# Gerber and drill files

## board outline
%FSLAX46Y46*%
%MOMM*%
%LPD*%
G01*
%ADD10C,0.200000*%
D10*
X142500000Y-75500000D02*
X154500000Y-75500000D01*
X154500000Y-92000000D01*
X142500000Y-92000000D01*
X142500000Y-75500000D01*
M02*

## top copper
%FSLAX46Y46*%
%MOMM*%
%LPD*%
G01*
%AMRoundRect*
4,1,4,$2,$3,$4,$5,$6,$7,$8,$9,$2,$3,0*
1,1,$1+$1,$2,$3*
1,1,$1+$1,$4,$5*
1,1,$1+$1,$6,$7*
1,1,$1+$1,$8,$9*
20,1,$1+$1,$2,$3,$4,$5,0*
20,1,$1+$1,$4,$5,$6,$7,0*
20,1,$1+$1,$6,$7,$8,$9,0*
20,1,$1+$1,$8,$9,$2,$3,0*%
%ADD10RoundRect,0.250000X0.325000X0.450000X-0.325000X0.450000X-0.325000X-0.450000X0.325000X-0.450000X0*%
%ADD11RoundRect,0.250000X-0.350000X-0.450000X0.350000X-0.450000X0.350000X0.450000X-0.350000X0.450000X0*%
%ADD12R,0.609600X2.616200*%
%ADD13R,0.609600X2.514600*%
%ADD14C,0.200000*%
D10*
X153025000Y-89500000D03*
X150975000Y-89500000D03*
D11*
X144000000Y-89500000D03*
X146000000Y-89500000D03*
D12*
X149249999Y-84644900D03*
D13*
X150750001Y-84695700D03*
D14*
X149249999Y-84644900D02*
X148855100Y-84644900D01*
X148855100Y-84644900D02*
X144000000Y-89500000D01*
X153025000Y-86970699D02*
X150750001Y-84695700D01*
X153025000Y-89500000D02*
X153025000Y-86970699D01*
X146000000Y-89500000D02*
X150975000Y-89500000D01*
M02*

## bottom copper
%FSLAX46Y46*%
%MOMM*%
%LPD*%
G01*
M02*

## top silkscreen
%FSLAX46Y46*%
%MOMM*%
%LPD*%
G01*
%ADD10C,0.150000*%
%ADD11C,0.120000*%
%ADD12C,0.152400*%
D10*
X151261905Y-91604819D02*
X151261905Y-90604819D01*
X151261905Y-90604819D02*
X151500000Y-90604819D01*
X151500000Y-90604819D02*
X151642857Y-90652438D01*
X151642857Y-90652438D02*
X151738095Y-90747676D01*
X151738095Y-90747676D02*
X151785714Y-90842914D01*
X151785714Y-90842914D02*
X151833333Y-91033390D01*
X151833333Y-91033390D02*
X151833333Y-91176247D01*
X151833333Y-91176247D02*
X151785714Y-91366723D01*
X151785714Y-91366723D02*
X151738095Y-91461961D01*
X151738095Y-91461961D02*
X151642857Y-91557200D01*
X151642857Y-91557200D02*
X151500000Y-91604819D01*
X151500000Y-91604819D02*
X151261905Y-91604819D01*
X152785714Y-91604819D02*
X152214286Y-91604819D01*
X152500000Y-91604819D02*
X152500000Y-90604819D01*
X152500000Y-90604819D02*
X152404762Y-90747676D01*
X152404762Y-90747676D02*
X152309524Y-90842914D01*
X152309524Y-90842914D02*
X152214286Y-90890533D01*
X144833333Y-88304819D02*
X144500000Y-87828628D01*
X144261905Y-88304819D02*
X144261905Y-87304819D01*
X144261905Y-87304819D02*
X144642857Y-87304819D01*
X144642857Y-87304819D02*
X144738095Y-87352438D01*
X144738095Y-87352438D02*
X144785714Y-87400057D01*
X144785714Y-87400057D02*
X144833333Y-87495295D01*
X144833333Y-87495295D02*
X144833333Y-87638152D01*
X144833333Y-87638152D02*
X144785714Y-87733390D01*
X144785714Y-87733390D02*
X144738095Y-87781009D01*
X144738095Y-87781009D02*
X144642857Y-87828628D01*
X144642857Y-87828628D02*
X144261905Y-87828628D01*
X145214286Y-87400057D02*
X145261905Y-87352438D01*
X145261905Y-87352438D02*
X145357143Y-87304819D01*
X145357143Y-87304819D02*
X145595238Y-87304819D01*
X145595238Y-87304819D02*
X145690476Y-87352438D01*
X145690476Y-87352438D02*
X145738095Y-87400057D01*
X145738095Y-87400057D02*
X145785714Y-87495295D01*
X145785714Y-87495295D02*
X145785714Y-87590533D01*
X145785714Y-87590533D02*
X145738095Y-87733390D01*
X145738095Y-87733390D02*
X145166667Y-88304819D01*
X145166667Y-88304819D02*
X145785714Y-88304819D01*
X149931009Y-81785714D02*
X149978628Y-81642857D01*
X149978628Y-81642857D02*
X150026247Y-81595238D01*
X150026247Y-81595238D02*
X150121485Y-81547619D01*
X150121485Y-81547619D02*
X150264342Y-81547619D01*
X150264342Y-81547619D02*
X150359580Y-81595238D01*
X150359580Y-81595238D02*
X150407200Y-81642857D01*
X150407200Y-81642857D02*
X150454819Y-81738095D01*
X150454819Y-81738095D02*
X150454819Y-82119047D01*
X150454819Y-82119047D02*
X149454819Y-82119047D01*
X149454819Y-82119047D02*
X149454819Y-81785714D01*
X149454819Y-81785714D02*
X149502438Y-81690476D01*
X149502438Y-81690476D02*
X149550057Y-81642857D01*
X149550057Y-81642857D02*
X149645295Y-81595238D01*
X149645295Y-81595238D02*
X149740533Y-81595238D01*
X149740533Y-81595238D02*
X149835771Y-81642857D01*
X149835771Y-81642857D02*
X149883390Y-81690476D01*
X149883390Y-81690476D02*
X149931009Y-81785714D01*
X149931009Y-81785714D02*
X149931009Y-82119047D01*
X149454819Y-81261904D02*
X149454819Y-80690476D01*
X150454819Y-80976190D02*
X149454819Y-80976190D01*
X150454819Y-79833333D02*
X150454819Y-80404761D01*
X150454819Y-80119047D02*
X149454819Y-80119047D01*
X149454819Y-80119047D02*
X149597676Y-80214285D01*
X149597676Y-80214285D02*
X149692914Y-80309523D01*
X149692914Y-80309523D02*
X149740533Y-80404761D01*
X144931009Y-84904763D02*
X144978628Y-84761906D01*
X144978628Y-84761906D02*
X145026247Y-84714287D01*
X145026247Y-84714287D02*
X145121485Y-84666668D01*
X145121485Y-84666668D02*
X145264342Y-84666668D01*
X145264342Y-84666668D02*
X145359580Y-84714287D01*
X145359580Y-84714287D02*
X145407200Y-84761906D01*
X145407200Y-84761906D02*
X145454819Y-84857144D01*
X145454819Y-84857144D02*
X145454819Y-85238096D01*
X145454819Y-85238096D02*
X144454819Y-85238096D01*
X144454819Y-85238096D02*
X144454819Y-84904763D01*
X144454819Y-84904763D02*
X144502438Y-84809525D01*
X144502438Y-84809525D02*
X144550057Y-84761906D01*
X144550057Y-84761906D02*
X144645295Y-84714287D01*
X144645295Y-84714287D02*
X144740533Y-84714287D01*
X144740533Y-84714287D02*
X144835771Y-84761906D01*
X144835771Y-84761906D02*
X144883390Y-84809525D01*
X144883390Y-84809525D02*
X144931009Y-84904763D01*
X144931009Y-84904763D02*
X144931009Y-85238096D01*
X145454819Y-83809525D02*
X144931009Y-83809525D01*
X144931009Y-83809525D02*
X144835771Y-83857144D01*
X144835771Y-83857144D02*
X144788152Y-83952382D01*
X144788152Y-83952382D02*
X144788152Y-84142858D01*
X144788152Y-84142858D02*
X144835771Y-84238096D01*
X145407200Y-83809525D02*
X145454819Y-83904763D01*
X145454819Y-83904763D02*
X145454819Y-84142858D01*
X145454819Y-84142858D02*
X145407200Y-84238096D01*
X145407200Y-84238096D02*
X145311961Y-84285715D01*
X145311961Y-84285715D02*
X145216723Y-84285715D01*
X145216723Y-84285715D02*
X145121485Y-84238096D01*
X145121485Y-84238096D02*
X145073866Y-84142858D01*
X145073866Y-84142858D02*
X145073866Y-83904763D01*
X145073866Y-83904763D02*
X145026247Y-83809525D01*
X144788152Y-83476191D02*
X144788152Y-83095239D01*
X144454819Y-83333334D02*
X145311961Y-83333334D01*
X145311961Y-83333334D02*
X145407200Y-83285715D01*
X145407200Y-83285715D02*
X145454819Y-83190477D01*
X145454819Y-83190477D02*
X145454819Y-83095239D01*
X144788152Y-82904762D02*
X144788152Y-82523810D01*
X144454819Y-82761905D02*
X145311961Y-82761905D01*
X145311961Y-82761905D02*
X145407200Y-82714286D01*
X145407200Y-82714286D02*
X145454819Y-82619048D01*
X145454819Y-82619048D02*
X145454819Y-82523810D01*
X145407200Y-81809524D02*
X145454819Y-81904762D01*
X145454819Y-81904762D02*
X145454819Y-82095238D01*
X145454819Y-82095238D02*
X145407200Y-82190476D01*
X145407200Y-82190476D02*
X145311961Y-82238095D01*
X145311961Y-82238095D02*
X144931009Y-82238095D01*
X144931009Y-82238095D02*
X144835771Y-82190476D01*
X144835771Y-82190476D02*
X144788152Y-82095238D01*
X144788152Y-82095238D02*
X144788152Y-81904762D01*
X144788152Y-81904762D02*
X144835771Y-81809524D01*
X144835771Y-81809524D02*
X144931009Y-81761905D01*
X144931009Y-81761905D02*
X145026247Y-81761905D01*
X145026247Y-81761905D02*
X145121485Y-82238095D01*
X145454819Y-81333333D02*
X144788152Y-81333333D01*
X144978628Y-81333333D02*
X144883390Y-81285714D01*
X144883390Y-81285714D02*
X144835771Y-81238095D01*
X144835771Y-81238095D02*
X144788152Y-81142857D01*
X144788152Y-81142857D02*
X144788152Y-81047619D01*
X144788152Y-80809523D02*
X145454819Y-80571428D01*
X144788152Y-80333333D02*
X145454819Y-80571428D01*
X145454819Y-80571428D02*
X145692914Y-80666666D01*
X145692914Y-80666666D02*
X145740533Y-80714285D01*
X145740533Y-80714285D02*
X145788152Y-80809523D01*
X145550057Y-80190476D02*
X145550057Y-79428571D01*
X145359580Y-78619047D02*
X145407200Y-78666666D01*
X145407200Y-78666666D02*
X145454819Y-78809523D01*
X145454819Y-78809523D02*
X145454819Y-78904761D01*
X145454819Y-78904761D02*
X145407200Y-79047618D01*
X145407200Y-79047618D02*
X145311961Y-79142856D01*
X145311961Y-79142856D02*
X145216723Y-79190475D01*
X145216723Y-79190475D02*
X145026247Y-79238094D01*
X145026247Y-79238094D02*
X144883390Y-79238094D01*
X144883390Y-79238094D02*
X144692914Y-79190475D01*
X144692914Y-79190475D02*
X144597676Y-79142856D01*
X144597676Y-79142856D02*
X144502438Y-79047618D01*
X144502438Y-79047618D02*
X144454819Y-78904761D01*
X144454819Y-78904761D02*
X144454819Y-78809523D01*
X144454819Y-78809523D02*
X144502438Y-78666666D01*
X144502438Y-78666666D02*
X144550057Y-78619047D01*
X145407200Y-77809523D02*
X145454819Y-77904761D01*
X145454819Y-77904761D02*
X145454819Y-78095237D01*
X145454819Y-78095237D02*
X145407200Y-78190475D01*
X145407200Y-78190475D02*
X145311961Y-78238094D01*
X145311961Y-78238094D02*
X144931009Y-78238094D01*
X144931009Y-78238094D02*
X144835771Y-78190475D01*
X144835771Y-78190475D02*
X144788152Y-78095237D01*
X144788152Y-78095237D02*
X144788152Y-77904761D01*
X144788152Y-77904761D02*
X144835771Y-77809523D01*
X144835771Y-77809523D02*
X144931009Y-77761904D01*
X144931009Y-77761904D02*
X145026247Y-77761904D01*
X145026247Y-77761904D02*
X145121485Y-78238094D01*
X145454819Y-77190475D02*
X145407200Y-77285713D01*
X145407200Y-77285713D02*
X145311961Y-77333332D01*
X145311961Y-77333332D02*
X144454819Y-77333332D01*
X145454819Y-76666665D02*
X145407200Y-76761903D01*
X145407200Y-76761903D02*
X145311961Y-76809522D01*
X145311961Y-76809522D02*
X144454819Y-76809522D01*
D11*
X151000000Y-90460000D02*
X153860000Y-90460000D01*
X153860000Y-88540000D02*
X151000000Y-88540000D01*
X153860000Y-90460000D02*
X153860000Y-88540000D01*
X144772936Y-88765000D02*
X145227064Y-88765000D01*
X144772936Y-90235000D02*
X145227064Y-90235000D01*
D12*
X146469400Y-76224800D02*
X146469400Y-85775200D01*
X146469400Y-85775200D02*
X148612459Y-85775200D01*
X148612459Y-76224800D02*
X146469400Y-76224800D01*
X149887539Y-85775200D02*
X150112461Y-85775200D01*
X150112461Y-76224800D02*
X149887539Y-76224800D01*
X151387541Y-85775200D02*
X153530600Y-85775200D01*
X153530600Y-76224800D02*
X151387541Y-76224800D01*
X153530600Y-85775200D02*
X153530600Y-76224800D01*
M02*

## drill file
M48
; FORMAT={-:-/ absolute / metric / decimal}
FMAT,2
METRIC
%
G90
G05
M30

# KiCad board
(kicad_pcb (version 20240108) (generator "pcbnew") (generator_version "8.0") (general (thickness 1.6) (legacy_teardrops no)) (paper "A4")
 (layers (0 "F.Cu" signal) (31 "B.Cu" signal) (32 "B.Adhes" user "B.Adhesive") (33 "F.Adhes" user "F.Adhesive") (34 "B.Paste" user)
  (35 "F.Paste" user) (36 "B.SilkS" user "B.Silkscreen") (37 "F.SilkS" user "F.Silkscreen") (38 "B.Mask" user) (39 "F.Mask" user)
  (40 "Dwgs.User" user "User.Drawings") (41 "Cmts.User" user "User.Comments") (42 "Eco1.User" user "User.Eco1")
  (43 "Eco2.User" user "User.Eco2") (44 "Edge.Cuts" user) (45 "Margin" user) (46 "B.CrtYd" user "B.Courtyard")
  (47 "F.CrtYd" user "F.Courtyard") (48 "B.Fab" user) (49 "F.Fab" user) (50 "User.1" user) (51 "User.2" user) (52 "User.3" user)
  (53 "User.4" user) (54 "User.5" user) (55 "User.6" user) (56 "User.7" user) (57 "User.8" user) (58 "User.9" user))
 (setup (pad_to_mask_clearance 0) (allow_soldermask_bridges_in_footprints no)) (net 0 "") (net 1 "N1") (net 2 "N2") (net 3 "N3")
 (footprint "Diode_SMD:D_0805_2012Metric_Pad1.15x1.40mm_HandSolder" (layer "F.Cu") (at 152 89.5 180)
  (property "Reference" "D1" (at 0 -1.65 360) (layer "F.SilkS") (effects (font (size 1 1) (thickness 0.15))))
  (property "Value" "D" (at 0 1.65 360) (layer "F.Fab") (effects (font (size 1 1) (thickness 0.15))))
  (fp_line (start 1 -0.96) (end -1.86 -0.96) (stroke (width 0.12) (type solid)) (layer "F.SilkS"))
  (fp_line (start -1.86 0.96) (end 1 0.96) (stroke (width 0.12) (type solid)) (layer "F.SilkS"))
  (fp_line (start -1.86 -0.96) (end -1.86 0.96) (stroke (width 0.12) (type solid)) (layer "F.SilkS"))
  (pad "1" smd roundrect (at -1.025 0 180) (size 1.15 1.4) (layers "F.Cu" "F.Paste" "F.Mask") (roundrect_rratio 0.217391) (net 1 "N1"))
  (pad "2" smd roundrect (at 1.025 0 180) (size 1.15 1.4) (layers "F.Cu" "F.Paste" "F.Mask") (roundrect_rratio 0.217391) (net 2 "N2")))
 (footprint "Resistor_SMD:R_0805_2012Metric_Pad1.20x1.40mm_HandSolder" (layer "F.Cu") (at 145 89.5)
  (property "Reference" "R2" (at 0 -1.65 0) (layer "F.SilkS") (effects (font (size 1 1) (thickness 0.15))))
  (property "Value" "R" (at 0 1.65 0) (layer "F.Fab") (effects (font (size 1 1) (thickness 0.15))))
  (fp_line (start -0.227064 -0.735) (end 0.227064 -0.735) (stroke (width 0.12) (type solid)) (layer "F.SilkS"))
  (fp_line (start -0.227064 0.735) (end 0.227064 0.735) (stroke (width 0.12) (type solid)) (layer "F.SilkS"))
  (pad "1" smd roundrect (at -1 0) (size 1.2 1.4) (layers "F.Cu" "F.Paste" "F.Mask") (roundrect_rratio 0.208333) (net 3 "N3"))
  (pad "2" smd roundrect (at 1 0) (size 1.2 1.4) (layers "F.Cu" "F.Paste" "F.Mask") (roundrect_rratio 0.208333) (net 2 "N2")))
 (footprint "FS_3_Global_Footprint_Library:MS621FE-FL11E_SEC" (layer "F.Cu") (at 150 81 90)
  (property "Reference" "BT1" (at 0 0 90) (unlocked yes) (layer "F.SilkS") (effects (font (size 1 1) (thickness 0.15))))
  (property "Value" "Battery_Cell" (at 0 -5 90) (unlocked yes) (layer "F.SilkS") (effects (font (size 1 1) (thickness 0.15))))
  (fp_line (start 4.7752 -3.5306) (end -4.7752 -3.5306) (stroke (width 0.1524) (type solid)) (layer "F.SilkS"))
  (fp_line (start -4.7752 -3.5306) (end -4.7752 -1.387541) (stroke (width 0.1524) (type solid)) (layer "F.SilkS"))
  (fp_line (start 4.7752 -1.387541) (end 4.7752 -3.5306) (stroke (width 0.1524) (type solid)) (layer "F.SilkS"))
  (fp_line (start -4.7752 -0.112461) (end -4.7752 0.112461) (stroke (width 0.1524) (type solid)) (layer "F.SilkS"))
  (fp_line (start 4.7752 0.112461) (end 4.7752 -0.112461) (stroke (width 0.1524) (type solid)) (layer "F.SilkS"))
  (fp_line (start -4.7752 1.387541) (end -4.7752 3.5306) (stroke (width 0.1524) (type solid)) (layer "F.SilkS"))
  (fp_line (start 4.7752 3.5306) (end 4.7752 1.387541) (stroke (width 0.1524) (type solid)) (layer "F.SilkS"))
  (fp_line (start -4.7752 3.5306) (end 4.7752 3.5306) (stroke (width 0.1524) (type solid)) (layer "F.SilkS"))
  (pad "1" smd rect (at -3.6449 -0.750001 90) (size 2.6162 0.6096) (layers "F.Cu" "F.Paste" "F.Mask") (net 3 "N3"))
  (pad "2" smd rect (at -3.6957 0.750001 90) (size 2.5146 0.6096) (layers "F.Cu" "F.Paste" "F.Mask") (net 1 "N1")))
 (gr_rect (start 142.5 75.5) (end 154.5 92) (stroke (width 0.2) (type default)) (fill none) (layer "Edge.Cuts"))
 (segment (start 149.249999 84.6449) (end 148.8551 84.6449) (width 0.2) (layer "F.Cu") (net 3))
 (segment (start 148.8551 84.6449) (end 144 89.5) (width 0.2) (layer "F.Cu") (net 3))
 (segment (start 153.025 86.970699) (end 150.750001 84.6957) (width 0.2) (layer "F.Cu") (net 1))
 (segment (start 153.025 89.5) (end 153.025 86.970699) (width 0.2) (layer "F.Cu") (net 1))
 (segment (start 146 89.5) (end 150.975 89.5) (width 0.2) (layer "F.Cu") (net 2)))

